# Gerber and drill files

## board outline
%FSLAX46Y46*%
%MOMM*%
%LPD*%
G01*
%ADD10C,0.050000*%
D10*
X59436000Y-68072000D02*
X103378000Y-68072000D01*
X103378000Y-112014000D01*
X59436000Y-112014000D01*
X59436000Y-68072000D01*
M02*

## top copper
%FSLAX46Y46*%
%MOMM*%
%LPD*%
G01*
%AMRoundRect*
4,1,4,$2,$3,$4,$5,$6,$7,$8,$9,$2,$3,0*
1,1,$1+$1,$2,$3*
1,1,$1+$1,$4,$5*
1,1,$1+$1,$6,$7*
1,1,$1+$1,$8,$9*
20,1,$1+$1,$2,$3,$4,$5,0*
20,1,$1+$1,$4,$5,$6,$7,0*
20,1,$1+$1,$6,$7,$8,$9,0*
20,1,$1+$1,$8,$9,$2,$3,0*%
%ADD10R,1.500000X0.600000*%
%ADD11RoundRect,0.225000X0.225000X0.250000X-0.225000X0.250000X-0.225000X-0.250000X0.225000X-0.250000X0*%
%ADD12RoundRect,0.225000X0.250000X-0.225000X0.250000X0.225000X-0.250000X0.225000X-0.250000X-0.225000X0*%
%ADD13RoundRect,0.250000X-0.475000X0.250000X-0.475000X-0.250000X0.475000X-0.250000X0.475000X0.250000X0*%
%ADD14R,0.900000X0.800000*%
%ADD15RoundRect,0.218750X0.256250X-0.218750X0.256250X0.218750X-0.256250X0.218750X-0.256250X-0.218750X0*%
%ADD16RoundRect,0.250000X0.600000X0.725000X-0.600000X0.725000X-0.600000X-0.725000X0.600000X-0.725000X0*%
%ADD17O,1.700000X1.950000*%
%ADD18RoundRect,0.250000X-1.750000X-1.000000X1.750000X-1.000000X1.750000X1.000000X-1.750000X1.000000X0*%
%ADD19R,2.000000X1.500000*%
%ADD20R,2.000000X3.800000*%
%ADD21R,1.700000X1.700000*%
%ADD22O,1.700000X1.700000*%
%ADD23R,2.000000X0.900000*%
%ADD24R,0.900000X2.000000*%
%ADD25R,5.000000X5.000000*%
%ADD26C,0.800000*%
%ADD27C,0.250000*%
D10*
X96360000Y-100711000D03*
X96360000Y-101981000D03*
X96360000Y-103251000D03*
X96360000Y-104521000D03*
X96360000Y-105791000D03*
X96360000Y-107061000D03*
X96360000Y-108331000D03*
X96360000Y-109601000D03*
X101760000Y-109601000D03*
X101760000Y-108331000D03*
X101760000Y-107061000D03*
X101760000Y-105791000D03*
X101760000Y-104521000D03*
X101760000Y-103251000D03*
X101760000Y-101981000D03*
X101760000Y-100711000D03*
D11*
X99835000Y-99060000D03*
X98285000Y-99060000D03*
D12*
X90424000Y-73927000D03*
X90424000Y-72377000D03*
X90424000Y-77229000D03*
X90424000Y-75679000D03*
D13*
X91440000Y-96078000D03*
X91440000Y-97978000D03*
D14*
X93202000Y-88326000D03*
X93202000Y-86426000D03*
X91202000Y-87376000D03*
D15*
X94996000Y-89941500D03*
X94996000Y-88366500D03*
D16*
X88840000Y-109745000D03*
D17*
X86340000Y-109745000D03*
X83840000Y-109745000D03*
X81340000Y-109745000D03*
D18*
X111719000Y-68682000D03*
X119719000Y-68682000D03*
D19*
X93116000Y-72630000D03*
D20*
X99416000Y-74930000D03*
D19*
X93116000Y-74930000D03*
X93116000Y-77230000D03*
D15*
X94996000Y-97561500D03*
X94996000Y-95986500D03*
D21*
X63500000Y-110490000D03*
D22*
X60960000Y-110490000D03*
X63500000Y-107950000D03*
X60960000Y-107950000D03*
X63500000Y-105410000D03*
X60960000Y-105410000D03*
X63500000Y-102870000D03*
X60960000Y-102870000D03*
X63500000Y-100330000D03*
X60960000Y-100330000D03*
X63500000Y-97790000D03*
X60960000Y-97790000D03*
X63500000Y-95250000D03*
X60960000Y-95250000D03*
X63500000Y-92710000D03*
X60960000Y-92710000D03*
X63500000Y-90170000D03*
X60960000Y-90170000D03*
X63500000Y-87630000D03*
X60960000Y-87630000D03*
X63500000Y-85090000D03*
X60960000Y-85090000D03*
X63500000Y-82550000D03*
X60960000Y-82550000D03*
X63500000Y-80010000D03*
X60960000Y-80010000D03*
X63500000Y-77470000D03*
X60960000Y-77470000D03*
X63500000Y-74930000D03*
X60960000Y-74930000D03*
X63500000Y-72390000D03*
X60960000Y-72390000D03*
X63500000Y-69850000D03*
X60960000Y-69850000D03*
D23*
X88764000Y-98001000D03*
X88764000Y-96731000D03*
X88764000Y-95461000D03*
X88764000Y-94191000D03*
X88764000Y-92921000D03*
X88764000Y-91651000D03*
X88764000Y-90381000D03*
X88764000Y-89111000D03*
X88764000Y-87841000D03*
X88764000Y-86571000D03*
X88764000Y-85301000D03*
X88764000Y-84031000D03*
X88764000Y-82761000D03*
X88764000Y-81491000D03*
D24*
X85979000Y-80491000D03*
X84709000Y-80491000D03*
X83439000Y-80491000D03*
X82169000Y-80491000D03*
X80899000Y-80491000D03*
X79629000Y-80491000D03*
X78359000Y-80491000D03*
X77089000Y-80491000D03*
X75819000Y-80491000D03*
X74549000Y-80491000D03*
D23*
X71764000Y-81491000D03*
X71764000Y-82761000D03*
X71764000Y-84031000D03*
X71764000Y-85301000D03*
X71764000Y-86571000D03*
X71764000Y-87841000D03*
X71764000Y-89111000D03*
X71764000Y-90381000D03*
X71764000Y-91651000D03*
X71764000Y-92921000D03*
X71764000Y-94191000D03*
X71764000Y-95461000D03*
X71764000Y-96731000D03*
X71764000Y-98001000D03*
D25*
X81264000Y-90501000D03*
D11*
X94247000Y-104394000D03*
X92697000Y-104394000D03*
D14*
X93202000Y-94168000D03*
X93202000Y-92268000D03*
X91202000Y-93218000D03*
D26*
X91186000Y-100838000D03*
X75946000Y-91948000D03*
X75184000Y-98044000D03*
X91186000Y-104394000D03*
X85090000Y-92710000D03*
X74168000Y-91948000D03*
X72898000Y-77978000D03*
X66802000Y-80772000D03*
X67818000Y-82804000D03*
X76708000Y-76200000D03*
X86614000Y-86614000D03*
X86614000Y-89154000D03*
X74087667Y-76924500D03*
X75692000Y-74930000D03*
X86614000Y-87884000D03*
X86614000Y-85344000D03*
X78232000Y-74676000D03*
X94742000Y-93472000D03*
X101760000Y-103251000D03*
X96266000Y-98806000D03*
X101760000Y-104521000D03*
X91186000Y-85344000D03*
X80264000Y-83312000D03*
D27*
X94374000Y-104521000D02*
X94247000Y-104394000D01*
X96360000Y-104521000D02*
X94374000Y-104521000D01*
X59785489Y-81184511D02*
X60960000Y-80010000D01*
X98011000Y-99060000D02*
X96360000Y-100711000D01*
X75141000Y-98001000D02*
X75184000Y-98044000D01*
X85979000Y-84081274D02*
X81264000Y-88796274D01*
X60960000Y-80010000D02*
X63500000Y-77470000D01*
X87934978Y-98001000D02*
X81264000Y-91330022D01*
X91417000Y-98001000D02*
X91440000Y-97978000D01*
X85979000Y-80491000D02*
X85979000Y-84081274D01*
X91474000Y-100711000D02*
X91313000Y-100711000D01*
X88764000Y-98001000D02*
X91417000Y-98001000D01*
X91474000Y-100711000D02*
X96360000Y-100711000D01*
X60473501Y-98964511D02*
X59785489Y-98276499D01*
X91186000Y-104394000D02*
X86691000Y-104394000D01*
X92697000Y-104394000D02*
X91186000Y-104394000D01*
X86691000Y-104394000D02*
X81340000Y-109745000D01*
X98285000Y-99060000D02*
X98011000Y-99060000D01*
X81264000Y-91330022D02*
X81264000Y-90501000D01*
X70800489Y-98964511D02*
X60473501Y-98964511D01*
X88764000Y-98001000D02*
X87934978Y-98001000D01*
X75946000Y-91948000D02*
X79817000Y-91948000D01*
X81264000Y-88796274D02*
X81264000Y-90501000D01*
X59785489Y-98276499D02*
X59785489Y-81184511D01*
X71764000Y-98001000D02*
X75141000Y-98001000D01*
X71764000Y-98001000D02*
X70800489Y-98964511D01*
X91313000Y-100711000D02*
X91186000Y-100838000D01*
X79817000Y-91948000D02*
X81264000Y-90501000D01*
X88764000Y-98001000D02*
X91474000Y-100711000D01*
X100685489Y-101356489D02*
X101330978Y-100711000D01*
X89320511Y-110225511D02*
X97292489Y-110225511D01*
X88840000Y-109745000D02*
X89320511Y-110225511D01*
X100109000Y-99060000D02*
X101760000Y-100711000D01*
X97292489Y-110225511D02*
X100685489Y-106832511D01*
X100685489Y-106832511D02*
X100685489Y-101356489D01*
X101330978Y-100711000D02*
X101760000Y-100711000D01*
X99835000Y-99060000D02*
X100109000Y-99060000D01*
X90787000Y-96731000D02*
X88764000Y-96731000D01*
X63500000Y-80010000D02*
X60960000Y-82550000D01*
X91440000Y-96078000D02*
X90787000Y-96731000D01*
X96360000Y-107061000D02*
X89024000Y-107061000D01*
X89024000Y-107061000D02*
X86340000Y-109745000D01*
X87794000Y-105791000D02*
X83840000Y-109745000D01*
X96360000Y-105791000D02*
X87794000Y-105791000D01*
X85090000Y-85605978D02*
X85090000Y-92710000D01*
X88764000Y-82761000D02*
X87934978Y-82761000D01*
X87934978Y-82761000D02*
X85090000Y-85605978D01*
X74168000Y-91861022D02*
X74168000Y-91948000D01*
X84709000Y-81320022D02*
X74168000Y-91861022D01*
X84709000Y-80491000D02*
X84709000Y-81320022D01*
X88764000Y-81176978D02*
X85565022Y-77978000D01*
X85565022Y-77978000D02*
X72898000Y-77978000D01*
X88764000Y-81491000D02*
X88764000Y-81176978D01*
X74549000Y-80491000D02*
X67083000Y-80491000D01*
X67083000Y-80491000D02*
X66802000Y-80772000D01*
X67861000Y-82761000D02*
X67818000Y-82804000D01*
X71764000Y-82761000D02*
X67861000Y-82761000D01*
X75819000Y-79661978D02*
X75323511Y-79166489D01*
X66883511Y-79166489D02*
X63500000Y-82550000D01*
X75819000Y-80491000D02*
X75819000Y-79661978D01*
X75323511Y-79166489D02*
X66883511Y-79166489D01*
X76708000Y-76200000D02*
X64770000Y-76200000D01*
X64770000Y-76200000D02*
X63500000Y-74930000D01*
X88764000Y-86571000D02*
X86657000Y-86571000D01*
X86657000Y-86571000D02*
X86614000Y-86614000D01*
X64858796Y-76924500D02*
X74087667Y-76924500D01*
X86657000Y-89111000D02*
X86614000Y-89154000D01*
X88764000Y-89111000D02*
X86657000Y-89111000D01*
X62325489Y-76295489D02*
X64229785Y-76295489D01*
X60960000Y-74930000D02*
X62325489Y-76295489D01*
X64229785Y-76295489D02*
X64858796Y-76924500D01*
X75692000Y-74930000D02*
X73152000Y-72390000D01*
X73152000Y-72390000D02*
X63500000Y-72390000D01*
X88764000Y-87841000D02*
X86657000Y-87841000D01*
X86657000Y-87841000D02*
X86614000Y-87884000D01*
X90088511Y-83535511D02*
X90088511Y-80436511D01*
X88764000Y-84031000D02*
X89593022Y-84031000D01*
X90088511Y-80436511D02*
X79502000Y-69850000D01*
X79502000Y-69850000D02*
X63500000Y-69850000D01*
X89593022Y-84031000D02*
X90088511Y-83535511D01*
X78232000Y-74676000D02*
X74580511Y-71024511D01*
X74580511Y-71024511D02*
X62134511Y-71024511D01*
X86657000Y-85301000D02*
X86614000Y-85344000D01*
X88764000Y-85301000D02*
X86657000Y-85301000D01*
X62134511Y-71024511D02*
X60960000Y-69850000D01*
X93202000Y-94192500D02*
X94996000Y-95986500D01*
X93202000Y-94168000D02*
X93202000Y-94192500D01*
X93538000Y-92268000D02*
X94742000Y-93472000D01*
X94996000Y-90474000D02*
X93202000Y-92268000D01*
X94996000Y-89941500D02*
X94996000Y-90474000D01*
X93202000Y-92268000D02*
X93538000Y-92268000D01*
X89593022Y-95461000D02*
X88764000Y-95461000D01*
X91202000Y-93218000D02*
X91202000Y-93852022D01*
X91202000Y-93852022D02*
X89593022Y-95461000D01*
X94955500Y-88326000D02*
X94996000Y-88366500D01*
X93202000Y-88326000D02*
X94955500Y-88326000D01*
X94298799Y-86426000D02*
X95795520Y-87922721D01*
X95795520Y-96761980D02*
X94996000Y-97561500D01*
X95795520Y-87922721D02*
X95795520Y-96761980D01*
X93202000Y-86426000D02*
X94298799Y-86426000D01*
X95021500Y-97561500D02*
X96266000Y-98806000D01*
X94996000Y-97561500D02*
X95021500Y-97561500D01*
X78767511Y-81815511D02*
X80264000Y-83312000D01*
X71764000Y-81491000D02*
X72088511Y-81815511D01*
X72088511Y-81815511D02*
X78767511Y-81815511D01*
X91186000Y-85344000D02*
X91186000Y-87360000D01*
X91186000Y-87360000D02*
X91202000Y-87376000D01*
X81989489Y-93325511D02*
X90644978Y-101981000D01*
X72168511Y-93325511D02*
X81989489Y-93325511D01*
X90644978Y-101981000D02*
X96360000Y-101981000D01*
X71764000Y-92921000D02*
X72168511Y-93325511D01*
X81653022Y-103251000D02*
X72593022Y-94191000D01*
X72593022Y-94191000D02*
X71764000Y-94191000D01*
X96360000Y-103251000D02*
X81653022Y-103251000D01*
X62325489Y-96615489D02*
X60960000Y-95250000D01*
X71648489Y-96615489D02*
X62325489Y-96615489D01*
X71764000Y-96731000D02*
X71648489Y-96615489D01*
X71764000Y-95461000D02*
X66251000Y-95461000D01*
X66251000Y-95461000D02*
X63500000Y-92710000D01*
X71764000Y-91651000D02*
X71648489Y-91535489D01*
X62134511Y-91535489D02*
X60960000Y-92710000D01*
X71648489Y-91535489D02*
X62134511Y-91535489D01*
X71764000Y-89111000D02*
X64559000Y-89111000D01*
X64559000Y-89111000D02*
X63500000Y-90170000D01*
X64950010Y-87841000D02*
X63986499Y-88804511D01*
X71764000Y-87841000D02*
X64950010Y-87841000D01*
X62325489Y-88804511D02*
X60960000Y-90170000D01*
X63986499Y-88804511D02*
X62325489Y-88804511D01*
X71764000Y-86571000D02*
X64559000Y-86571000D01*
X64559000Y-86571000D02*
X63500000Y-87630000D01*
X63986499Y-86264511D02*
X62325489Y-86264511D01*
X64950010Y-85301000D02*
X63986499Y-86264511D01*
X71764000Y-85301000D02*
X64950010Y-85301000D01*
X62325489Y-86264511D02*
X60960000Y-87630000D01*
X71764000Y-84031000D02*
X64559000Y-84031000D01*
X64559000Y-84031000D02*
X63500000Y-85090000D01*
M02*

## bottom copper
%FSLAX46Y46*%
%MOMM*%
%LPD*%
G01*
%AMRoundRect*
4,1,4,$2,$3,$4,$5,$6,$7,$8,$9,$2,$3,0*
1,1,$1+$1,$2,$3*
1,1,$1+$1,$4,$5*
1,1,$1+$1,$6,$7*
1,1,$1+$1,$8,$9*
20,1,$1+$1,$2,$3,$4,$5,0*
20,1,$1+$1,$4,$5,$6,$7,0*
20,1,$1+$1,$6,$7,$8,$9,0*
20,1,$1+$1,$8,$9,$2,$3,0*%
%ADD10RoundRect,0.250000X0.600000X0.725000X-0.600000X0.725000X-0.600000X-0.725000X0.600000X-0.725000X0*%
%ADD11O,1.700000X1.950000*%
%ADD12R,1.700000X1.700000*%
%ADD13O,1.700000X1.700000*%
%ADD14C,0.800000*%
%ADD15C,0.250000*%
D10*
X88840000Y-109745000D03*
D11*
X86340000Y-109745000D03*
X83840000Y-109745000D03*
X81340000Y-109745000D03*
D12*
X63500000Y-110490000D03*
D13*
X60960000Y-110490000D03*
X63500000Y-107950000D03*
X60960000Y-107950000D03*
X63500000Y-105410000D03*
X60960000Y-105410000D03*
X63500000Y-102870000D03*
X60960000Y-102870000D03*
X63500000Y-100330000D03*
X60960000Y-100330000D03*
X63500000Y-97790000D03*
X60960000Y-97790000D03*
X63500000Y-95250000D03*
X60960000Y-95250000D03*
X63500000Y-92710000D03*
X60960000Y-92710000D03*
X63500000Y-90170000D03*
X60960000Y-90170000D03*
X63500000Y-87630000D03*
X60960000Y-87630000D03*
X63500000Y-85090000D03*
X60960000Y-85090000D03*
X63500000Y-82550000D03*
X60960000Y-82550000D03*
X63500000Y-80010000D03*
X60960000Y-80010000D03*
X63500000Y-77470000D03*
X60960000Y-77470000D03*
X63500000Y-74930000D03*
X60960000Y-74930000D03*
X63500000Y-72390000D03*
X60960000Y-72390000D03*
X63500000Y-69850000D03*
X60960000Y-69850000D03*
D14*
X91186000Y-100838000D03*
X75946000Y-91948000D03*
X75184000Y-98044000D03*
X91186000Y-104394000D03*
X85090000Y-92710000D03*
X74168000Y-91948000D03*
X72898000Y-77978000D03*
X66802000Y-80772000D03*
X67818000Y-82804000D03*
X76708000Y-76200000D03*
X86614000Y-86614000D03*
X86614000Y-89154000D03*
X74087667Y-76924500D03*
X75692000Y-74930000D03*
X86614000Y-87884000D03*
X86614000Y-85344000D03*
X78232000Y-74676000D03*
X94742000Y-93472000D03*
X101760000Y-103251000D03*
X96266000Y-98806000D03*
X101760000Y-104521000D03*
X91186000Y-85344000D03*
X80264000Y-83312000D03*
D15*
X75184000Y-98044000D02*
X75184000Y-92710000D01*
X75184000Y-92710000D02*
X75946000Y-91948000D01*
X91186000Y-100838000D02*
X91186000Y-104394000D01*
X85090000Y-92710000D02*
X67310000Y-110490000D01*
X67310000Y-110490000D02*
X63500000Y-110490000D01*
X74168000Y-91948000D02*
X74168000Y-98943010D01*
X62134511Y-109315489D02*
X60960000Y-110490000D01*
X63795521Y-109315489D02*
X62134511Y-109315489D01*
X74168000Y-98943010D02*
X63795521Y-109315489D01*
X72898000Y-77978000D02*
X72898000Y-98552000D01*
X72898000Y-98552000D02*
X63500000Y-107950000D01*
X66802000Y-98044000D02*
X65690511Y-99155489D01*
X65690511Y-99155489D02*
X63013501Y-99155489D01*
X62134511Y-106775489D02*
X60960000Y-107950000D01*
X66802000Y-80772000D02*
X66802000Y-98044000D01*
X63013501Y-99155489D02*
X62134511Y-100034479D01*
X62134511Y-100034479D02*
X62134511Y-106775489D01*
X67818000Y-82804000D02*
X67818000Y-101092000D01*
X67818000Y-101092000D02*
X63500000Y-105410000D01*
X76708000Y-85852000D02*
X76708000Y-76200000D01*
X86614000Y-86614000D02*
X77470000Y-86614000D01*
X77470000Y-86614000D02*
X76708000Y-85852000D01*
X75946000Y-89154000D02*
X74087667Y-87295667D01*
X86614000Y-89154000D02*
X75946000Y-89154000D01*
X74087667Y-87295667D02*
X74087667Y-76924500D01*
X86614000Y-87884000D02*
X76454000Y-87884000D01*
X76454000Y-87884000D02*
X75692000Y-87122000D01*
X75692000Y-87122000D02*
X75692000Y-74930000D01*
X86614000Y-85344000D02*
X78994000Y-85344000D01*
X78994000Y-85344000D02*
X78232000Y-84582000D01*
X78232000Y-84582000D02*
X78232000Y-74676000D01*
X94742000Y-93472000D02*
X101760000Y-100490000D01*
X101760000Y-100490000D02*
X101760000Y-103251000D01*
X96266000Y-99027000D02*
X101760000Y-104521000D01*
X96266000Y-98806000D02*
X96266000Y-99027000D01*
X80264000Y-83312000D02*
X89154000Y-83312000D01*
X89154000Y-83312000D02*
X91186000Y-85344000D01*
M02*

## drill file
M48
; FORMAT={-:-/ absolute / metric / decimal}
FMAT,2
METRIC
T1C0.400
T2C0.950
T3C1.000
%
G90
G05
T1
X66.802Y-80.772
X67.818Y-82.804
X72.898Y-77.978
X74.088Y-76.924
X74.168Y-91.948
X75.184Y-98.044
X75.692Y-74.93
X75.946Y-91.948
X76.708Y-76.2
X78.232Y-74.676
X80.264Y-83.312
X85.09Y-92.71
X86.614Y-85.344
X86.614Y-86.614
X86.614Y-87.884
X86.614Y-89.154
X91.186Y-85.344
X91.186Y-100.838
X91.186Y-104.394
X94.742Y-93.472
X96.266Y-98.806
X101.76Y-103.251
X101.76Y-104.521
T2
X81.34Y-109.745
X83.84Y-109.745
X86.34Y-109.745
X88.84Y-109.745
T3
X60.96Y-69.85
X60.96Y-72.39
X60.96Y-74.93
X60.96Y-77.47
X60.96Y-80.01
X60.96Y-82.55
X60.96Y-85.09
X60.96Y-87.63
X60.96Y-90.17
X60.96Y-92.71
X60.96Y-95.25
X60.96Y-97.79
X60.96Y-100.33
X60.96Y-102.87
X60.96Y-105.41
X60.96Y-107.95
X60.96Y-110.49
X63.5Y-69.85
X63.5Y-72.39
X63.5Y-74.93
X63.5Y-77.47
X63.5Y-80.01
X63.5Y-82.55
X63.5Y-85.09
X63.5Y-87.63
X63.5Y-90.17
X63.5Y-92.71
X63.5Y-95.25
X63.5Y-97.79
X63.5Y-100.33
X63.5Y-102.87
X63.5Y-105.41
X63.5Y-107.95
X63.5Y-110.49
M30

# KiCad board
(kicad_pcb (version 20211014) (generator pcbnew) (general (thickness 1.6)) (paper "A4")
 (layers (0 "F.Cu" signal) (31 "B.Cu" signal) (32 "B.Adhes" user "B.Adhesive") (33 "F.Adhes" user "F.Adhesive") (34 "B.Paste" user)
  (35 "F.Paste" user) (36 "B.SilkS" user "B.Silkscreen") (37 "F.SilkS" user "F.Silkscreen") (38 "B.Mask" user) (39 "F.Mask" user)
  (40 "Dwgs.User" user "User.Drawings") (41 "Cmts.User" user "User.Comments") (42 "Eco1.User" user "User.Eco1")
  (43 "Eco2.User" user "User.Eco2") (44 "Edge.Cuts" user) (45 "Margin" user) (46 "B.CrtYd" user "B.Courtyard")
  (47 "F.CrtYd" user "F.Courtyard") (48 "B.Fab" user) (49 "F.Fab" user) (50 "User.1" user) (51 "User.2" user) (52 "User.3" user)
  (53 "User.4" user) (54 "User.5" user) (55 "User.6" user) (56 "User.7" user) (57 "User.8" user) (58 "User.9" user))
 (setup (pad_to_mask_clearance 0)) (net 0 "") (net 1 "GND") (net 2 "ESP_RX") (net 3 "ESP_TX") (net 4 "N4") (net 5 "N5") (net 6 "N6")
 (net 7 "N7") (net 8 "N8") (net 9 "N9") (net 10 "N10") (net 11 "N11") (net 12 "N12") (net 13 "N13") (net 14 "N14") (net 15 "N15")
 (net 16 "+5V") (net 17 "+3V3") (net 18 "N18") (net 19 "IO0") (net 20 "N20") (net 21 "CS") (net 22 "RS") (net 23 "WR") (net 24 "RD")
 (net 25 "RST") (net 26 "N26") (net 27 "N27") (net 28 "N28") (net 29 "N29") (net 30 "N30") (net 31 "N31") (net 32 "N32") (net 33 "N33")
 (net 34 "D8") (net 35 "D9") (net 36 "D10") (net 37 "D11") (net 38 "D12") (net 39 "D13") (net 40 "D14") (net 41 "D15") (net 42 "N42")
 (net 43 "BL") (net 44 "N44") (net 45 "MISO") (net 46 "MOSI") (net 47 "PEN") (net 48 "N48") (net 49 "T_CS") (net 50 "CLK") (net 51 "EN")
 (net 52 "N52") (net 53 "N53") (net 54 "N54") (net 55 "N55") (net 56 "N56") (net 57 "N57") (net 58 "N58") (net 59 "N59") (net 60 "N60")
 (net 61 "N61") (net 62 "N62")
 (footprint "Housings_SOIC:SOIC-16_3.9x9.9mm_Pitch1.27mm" (layer "F.Cu") (at 99.06 105.156)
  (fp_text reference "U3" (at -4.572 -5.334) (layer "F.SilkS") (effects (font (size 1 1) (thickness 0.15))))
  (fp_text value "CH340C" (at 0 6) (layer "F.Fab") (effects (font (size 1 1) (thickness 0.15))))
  (pad "1" smd rect locked (at -2.7 -4.445) (size 1.5 0.6) (layers "F.Cu" "F.Paste" "F.Mask") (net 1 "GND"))
  (pad "2" smd rect locked (at -2.7 -3.175) (size 1.5 0.6) (layers "F.Cu" "F.Paste" "F.Mask") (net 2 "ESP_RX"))
  (pad "3" smd rect locked (at -2.7 -1.905) (size 1.5 0.6) (layers "F.Cu" "F.Paste" "F.Mask") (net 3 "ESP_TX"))
  (pad "4" smd rect locked (at -2.7 -0.635) (size 1.5 0.6) (layers "F.Cu" "F.Paste" "F.Mask") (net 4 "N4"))
  (pad "5" smd rect locked (at -2.7 0.635) (size 1.5 0.6) (layers "F.Cu" "F.Paste" "F.Mask") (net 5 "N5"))
  (pad "6" smd rect locked (at -2.7 1.905) (size 1.5 0.6) (layers "F.Cu" "F.Paste" "F.Mask") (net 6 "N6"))
  (pad "7" smd rect locked (at -2.7 3.175) (size 1.5 0.6) (layers "F.Cu" "F.Paste" "F.Mask") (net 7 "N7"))
  (pad "8" smd rect locked (at -2.7 4.445) (size 1.5 0.6) (layers "F.Cu" "F.Paste" "F.Mask") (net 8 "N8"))
  (pad "9" smd rect locked (at 2.7 4.445) (size 1.5 0.6) (layers "F.Cu" "F.Paste" "F.Mask") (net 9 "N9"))
  (pad "10" smd rect locked (at 2.7 3.175) (size 1.5 0.6) (layers "F.Cu" "F.Paste" "F.Mask") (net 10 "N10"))
  (pad "11" smd rect locked (at 2.7 1.905) (size 1.5 0.6) (layers "F.Cu" "F.Paste" "F.Mask") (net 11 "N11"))
  (pad "12" smd rect locked (at 2.7 0.635) (size 1.5 0.6) (layers "F.Cu" "F.Paste" "F.Mask") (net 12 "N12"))
  (pad "13" smd rect locked (at 2.7 -0.635) (size 1.5 0.6) (layers "F.Cu" "F.Paste" "F.Mask") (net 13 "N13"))
  (pad "14" smd rect locked (at 2.7 -1.905) (size 1.5 0.6) (layers "F.Cu" "F.Paste" "F.Mask") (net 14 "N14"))
  (pad "15" smd rect locked (at 2.7 -3.175) (size 1.5 0.6) (layers "F.Cu" "F.Paste" "F.Mask") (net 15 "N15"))
  (pad "16" smd rect locked (at 2.7 -4.445) (size 1.5 0.6) (layers "F.Cu" "F.Paste" "F.Mask") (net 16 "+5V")))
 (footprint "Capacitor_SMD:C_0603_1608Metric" (layer "F.Cu") (at 99.06 99.06 180)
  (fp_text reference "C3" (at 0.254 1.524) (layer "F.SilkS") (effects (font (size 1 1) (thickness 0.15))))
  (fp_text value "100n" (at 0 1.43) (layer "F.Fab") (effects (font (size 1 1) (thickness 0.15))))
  (pad "1" smd roundrect locked (at -0.775 0 180) (size 0.9 0.95) (layers "F.Cu" "F.Paste" "F.Mask") (roundrect_rratio 0.25) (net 16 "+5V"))
  (pad "2" smd roundrect locked (at 0.775 0 180) (size 0.9 0.95) (layers "F.Cu" "F.Paste" "F.Mask") (roundrect_rratio 0.25) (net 1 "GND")))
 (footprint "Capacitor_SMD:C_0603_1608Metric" (layer "F.Cu") (at 90.424 73.152 90)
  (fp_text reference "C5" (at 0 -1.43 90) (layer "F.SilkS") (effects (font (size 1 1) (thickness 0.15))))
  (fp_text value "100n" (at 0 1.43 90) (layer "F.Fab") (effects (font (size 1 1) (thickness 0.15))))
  (pad "1" smd roundrect locked (at -0.775 0 90) (size 0.9 0.95) (layers "F.Cu" "F.Paste" "F.Mask") (roundrect_rratio 0.25) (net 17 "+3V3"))
  (pad "2" smd roundrect locked (at 0.775 0 90) (size 0.9 0.95) (layers "F.Cu" "F.Paste" "F.Mask") (roundrect_rratio 0.25) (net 1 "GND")))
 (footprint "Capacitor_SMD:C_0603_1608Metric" (layer "F.Cu") (at 90.424 76.454 90)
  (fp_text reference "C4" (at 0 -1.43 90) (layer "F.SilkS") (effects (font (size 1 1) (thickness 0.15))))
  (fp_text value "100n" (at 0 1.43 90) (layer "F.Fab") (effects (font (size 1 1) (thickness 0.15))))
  (pad "1" smd roundrect locked (at -0.775 0 90) (size 0.9 0.95) (layers "F.Cu" "F.Paste" "F.Mask") (roundrect_rratio 0.25) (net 16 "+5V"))
  (pad "2" smd roundrect locked (at 0.775 0 90) (size 0.9 0.95) (layers "F.Cu" "F.Paste" "F.Mask") (roundrect_rratio 0.25) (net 1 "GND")))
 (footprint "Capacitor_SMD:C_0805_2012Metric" (layer "F.Cu") (at 91.44 97.028 -90)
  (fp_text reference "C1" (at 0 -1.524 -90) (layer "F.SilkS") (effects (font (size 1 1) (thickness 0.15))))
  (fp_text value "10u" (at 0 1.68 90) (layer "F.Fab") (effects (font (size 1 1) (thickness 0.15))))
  (pad "1" smd roundrect locked (at -0.95 0 270) (size 1 1.45) (layers "F.Cu" "F.Paste" "F.Mask") (roundrect_rratio 0.25) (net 17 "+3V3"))
  (pad "2" smd roundrect locked (at 0.95 0 270) (size 1 1.45) (layers "F.Cu" "F.Paste" "F.Mask") (roundrect_rratio 0.25) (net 1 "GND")))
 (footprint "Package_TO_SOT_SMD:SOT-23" (layer "F.Cu") (at 92.202 87.376 180)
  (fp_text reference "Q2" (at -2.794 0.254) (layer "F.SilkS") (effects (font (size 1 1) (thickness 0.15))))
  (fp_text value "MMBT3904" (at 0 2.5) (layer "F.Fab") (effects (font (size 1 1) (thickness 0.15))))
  (pad "1" smd rect locked (at -1 -0.95 180) (size 0.9 0.8) (layers "F.Cu" "F.Paste" "F.Mask") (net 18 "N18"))
  (pad "2" smd rect locked (at -1 0.95 180) (size 0.9 0.8) (layers "F.Cu" "F.Paste" "F.Mask") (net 13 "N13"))
  (pad "3" smd rect locked (at 1 0 180) (size 0.9 0.8) (layers "F.Cu" "F.Paste" "F.Mask") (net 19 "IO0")))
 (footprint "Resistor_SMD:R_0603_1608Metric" (layer "F.Cu") (at 94.996 89.154 90)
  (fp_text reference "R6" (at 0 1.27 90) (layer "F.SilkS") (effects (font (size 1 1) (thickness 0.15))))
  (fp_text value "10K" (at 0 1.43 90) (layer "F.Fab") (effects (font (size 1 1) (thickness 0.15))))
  (pad "1" smd roundrect locked (at -0.7875 0 90) (size 0.875 0.95) (layers "F.Cu" "F.Paste" "F.Mask") (roundrect_rratio 0.25)
   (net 14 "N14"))
  (pad "2" smd roundrect locked (at 0.7875 0 90) (size 0.875 0.95) (layers "F.Cu" "F.Paste" "F.Mask") (roundrect_rratio 0.25) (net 18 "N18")))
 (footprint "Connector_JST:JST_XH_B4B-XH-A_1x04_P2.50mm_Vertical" (layer "F.Cu") (at 88.84 109.745 180)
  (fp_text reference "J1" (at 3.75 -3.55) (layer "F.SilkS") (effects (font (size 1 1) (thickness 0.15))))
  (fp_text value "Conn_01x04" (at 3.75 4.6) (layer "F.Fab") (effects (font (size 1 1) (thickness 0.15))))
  (pad "1" thru_hole roundrect (at 0 0 180) (size 1.7 1.95) (drill 0.95) (layers *.Cu *.Mask) (roundrect_rratio 0.147059) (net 16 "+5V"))
  (pad "2" thru_hole oval (at 2.5 0 180) (size 1.7 1.95) (drill 0.95) (layers *.Cu *.Mask) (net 6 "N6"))
  (pad "3" thru_hole oval (at 5 0 180) (size 1.7 1.95) (drill 0.95) (layers *.Cu *.Mask) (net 5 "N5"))
  (pad "4" thru_hole oval (at 7.5 0 180) (size 1.7 1.95) (drill 0.95) (layers *.Cu *.Mask) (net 1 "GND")))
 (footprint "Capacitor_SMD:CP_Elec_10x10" (layer "F.Cu") (at 115.719 68.682)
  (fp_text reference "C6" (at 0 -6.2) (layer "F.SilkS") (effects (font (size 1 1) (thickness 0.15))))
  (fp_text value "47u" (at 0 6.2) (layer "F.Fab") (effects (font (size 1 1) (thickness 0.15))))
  (pad "1" smd roundrect locked (at -4 0) (size 4 2.5) (layers "F.Cu" "F.Paste" "F.Mask") (roundrect_rratio 0.1) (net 16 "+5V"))
  (pad "2" smd roundrect locked (at 4 0) (size 4 2.5) (layers "F.Cu" "F.Paste" "F.Mask") (roundrect_rratio 0.1) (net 1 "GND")))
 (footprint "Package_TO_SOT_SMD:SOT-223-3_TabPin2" (layer "F.Cu") (at 96.266 74.93)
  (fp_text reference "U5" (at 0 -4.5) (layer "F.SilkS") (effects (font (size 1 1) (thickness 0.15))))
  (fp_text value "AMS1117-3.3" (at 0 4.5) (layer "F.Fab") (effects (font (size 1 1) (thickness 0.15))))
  (pad "1" smd rect locked (at -3.15 -2.3) (size 2 1.5) (layers "F.Cu" "F.Paste" "F.Mask") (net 1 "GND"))
  (pad "2" smd rect locked (at 3.15 0) (size 2 3.8) (layers "F.Cu" "F.Paste" "F.Mask") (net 17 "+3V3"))
  (pad "2" smd rect locked (at -3.15 0) (size 2 1.5) (layers "F.Cu" "F.Paste" "F.Mask") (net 17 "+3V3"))
  (pad "3" smd rect locked (at -3.15 2.3) (size 2 1.5) (layers "F.Cu" "F.Paste" "F.Mask") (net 16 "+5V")))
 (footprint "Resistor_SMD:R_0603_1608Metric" (layer "F.Cu") (at 94.996 96.774 90)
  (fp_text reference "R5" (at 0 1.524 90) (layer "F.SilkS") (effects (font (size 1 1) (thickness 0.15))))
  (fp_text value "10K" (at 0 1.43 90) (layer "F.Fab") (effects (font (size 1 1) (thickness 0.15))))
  (pad "1" smd roundrect locked (at -0.7875 0 90) (size 0.875 0.95) (layers "F.Cu" "F.Paste" "F.Mask") (roundrect_rratio 0.25)
   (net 13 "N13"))
  (pad "2" smd roundrect locked (at 0.7875 0 90) (size 0.875 0.95) (layers "F.Cu" "F.Paste" "F.Mask") (roundrect_rratio 0.25) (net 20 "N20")))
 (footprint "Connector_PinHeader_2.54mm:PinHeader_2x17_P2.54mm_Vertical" (layer "F.Cu") (at 63.5 110.49 180)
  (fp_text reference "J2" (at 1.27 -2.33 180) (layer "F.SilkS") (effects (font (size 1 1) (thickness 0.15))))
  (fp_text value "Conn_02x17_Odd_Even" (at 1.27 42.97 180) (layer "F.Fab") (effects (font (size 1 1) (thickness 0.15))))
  (pad "1" thru_hole rect locked (at 0 0 180) (size 1.7 1.7) (drill 1) (layers *.Cu *.Mask) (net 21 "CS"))
  (pad "2" thru_hole oval locked (at 2.54 0 180) (size 1.7 1.7) (drill 1) (layers *.Cu *.Mask) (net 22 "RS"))
  (pad "3" thru_hole oval locked (at 0 2.54 180) (size 1.7 1.7) (drill 1) (layers *.Cu *.Mask) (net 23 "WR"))
  (pad "4" thru_hole oval locked (at 2.54 2.54 180) (size 1.7 1.7) (drill 1) (layers *.Cu *.Mask) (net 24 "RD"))
  (pad "5" thru_hole oval locked (at 0 5.08 180) (size 1.7 1.7) (drill 1) (layers *.Cu *.Mask) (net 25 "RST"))
  (pad "6" thru_hole oval locked (at 2.54 5.08 180) (size 1.7 1.7) (drill 1) (layers *.Cu *.Mask) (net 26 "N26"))
  (pad "7" thru_hole oval locked (at 0 7.62 180) (size 1.7 1.7) (drill 1) (layers *.Cu *.Mask) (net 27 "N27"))
  (pad "8" thru_hole oval locked (at 2.54 7.62 180) (size 1.7 1.7) (drill 1) (layers *.Cu *.Mask) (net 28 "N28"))
  (pad "9" thru_hole oval locked (at 0 10.16 180) (size 1.7 1.7) (drill 1) (layers *.Cu *.Mask) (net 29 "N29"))
  (pad "10" thru_hole oval locked (at 2.54 10.16 180) (size 1.7 1.7) (drill 1) (layers *.Cu *.Mask) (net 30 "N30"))
  (pad "11" thru_hole oval locked (at 0 12.7 180) (size 1.7 1.7) (drill 1) (layers *.Cu *.Mask) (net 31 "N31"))
  (pad "12" thru_hole oval locked (at 2.54 12.7 180) (size 1.7 1.7) (drill 1) (layers *.Cu *.Mask) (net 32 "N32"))
  (pad "13" thru_hole oval locked (at 0 15.24 180) (size 1.7 1.7) (drill 1) (layers *.Cu *.Mask) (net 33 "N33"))
  (pad "14" thru_hole oval locked (at 2.54 15.24 180) (size 1.7 1.7) (drill 1) (layers *.Cu *.Mask) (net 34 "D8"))
  (pad "15" thru_hole oval locked (at 0 17.78 180) (size 1.7 1.7) (drill 1) (layers *.Cu *.Mask) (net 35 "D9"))
  (pad "16" thru_hole oval locked (at 2.54 17.78 180) (size 1.7 1.7) (drill 1) (layers *.Cu *.Mask) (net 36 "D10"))
  (pad "17" thru_hole oval locked (at 0 20.32 180) (size 1.7 1.7) (drill 1) (layers *.Cu *.Mask) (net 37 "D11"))
  (pad "18" thru_hole oval locked (at 2.54 20.32 180) (size 1.7 1.7) (drill 1) (layers *.Cu *.Mask) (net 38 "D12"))
  (pad "19" thru_hole oval locked (at 0 22.86 180) (size 1.7 1.7) (drill 1) (layers *.Cu *.Mask) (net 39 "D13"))
  (pad "20" thru_hole oval locked (at 2.54 22.86 180) (size 1.7 1.7) (drill 1) (layers *.Cu *.Mask) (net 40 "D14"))
  (pad "21" thru_hole oval locked (at 0 25.4 180) (size 1.7 1.7) (drill 1) (layers *.Cu *.Mask) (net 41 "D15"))
  (pad "22" thru_hole oval locked (at 2.54 25.4 180) (size 1.7 1.7) (drill 1) (layers *.Cu *.Mask) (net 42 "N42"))
  (pad "23" thru_hole oval locked (at 0 27.94 180) (size 1.7 1.7) (drill 1) (layers *.Cu *.Mask) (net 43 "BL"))
  (pad "24" thru_hole oval locked (at 2.54 27.94 180) (size 1.7 1.7) (drill 1) (layers *.Cu *.Mask) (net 17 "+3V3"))
  (pad "25" thru_hole oval locked (at 0 30.48 180) (size 1.7 1.7) (drill 1) (layers *.Cu *.Mask) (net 17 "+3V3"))
  (pad "26" thru_hole oval locked (at 2.54 30.48 180) (size 1.7 1.7) (drill 1) (layers *.Cu *.Mask) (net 1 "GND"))
  (pad "27" thru_hole oval locked (at 0 33.02 180) (size 1.7 1.7) (drill 1) (layers *.Cu *.Mask) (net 1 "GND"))
  (pad "28" thru_hole oval locked (at 2.54 33.02 180) (size 1.7 1.7) (drill 1) (layers *.Cu *.Mask) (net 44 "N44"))
  (pad "29" thru_hole oval locked (at 0 35.56 180) (size 1.7 1.7) (drill 1) (layers *.Cu *.Mask) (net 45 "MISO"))
  (pad "30" thru_hole oval locked (at 2.54 35.56 180) (size 1.7 1.7) (drill 1) (layers *.Cu *.Mask) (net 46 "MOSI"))
  (pad "31" thru_hole oval locked (at 0 38.1 180) (size 1.7 1.7) (drill 1) (layers *.Cu *.Mask) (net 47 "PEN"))
  (pad "32" thru_hole oval locked (at 2.54 38.1 180) (size 1.7 1.7) (drill 1) (layers *.Cu *.Mask) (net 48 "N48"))
  (pad "33" thru_hole oval locked (at 0 40.64 180) (size 1.7 1.7) (drill 1) (layers *.Cu *.Mask) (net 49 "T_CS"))
  (pad "34" thru_hole oval locked (at 2.54 40.64 180) (size 1.7 1.7) (drill 1) (layers *.Cu *.Mask) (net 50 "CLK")))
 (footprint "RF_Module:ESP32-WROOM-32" (layer "F.Cu") (at 80.264 89.746 180)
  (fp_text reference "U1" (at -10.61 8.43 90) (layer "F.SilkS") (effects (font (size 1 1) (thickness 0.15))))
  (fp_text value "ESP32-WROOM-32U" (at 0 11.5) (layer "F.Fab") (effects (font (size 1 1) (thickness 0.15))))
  (pad "1" smd rect locked (at -8.5 -8.255 180) (size 2 0.9) (layers "F.Cu" "F.Paste" "F.Mask") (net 1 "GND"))
  (pad "2" smd rect locked (at -8.5 -6.985 180) (size 2 0.9) (layers "F.Cu" "F.Paste" "F.Mask") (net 17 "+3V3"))
  (pad "3" smd rect locked (at -8.5 -5.715 180) (size 2 0.9) (layers "F.Cu" "F.Paste" "F.Mask") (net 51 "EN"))
  (pad "4" smd rect locked (at -8.5 -4.445 180) (size 2 0.9) (layers "F.Cu" "F.Paste" "F.Mask") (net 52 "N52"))
  (pad "5" smd rect locked (at -8.5 -3.175 180) (size 2 0.9) (layers "F.Cu" "F.Paste" "F.Mask") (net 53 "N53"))
  (pad "6" smd rect locked (at -8.5 -1.905 180) (size 2 0.9) (layers "F.Cu" "F.Paste" "F.Mask") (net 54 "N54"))
  (pad "7" smd rect locked (at -8.5 -0.635 180) (size 2 0.9) (layers "F.Cu" "F.Paste" "F.Mask") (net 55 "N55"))
  (pad "8" smd rect locked (at -8.5 0.635 180) (size 2 0.9) (layers "F.Cu" "F.Paste" "F.Mask") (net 46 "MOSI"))
  (pad "9" smd rect locked (at -8.5 1.905 180) (size 2 0.9) (layers "F.Cu" "F.Paste" "F.Mask") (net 47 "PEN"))
  (pad "10" smd rect locked (at -8.5 3.175 180) (size 2 0.9) (layers "F.Cu" "F.Paste" "F.Mask") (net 45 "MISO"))
  (pad "11" smd rect locked (at -8.5 4.445 180) (size 2 0.9) (layers "F.Cu" "F.Paste" "F.Mask") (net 50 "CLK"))
  (pad "12" smd rect locked (at -8.5 5.715 180) (size 2 0.9) (layers "F.Cu" "F.Paste" "F.Mask") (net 49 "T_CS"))
  (pad "13" smd rect locked (at -8.5 6.985 180) (size 2 0.9) (layers "F.Cu" "F.Paste" "F.Mask") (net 21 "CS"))
  (pad "14" smd rect locked (at -8.5 8.255 180) (size 2 0.9) (layers "F.Cu" "F.Paste" "F.Mask") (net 23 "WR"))
  (pad "15" smd rect locked (at -5.715 9.255 270) (size 2 0.9) (layers "F.Cu" "F.Paste" "F.Mask") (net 1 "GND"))
  (pad "16" smd rect locked (at -4.445 9.255 270) (size 2 0.9) (layers "F.Cu" "F.Paste" "F.Mask") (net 22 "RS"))
  (pad "17" smd rect locked (at -3.175 9.255 270) (size 2 0.9) (layers "F.Cu" "F.Paste" "F.Mask") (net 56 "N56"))
  (pad "18" smd rect locked (at -1.905 9.255 270) (size 2 0.9) (layers "F.Cu" "F.Paste" "F.Mask") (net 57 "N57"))
  (pad "19" smd rect locked (at -0.635 9.255 270) (size 2 0.9) (layers "F.Cu" "F.Paste" "F.Mask") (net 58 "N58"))
  (pad "20" smd rect locked (at 0.635 9.255 270) (size 2 0.9) (layers "F.Cu" "F.Paste" "F.Mask") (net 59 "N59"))
  (pad "21" smd rect locked (at 1.905 9.255 270) (size 2 0.9) (layers "F.Cu" "F.Paste" "F.Mask") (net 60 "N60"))
  (pad "22" smd rect locked (at 3.175 9.255 270) (size 2 0.9) (layers "F.Cu" "F.Paste" "F.Mask") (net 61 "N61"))
  (pad "23" smd rect locked (at 4.445 9.255 270) (size 2 0.9) (layers "F.Cu" "F.Paste" "F.Mask") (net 43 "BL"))
  (pad "24" smd rect locked (at 5.715 9.255 270) (size 2 0.9) (layers "F.Cu" "F.Paste" "F.Mask") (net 24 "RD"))
  (pad "25" smd rect locked (at 8.5 8.255 180) (size 2 0.9) (layers "F.Cu" "F.Paste" "F.Mask") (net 19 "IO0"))
  (pad "26" smd rect locked (at 8.5 6.985 180) (size 2 0.9) (layers "F.Cu" "F.Paste" "F.Mask") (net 25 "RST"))
  (pad "27" smd rect locked (at 8.5 5.715 180) (size 2 0.9) (layers "F.Cu" "F.Paste" "F.Mask") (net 41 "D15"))
  (pad "28" smd rect locked (at 8.5 4.445 180) (size 2 0.9) (layers "F.Cu" "F.Paste" "F.Mask") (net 40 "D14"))
  (pad "29" smd rect locked (at 8.5 3.175 180) (size 2 0.9) (layers "F.Cu" "F.Paste" "F.Mask") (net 39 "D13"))
  (pad "30" smd rect locked (at 8.5 1.905 180) (size 2 0.9) (layers "F.Cu" "F.Paste" "F.Mask") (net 38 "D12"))
  (pad "31" smd rect locked (at 8.5 0.635 180) (size 2 0.9) (layers "F.Cu" "F.Paste" "F.Mask") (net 37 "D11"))
  (pad "32" smd rect locked (at 8.5 -0.635 180) (size 2 0.9) (layers "F.Cu" "F.Paste" "F.Mask") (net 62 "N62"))
  (pad "33" smd rect locked (at 8.5 -1.905 180) (size 2 0.9) (layers "F.Cu" "F.Paste" "F.Mask") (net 36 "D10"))
  (pad "34" smd rect locked (at 8.5 -3.175 180) (size 2 0.9) (layers "F.Cu" "F.Paste" "F.Mask") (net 2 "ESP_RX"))
  (pad "35" smd rect locked (at 8.5 -4.445 180) (size 2 0.9) (layers "F.Cu" "F.Paste" "F.Mask") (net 3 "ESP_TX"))
  (pad "36" smd rect locked (at 8.5 -5.715 180) (size 2 0.9) (layers "F.Cu" "F.Paste" "F.Mask") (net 35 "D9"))
  (pad "37" smd rect locked (at 8.5 -6.985 180) (size 2 0.9) (layers "F.Cu" "F.Paste" "F.Mask") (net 34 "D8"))
  (pad "38" smd rect locked (at 8.5 -8.255 180) (size 2 0.9) (layers "F.Cu" "F.Paste" "F.Mask") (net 1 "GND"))
  (pad "39" smd rect locked (at -1 -0.755 180) (size 5 5) (layers "F.Cu" "F.Paste" "F.Mask") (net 1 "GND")))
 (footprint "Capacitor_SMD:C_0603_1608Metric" (layer "F.Cu") (at 93.472 104.394 180)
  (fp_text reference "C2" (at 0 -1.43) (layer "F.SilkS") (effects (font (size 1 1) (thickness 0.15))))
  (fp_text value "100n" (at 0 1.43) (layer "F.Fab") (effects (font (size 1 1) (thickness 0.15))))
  (pad "1" smd roundrect locked (at -0.775 0 180) (size 0.9 0.95) (layers "F.Cu" "F.Paste" "F.Mask") (roundrect_rratio 0.25) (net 4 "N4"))
  (pad "2" smd roundrect locked (at 0.775 0 180) (size 0.9 0.95) (layers "F.Cu" "F.Paste" "F.Mask") (roundrect_rratio 0.25) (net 1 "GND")))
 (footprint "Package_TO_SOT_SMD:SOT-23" (layer "F.Cu") (at 92.202 93.218 180)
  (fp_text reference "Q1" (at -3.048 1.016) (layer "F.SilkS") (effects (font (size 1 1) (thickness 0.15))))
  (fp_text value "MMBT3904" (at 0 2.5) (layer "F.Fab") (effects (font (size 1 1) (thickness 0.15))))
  (pad "1" smd rect locked (at -1 -0.95 180) (size 0.9 0.8) (layers "F.Cu" "F.Paste" "F.Mask") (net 20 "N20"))
  (pad "2" smd rect locked (at -1 0.95 180) (size 0.9 0.8) (layers "F.Cu" "F.Paste" "F.Mask") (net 14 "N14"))
  (pad "3" smd rect locked (at 1 0 180) (size 0.9 0.8) (layers "F.Cu" "F.Paste" "F.Mask") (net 51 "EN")))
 (gr_rect (start 59.436 112.014) (end 103.378 68.072) (layer "Edge.Cuts") (width 0.05) (fill none))
 (segment (start 94.374 104.521) (end 94.247 104.394) (width 0.25) (layer "F.Cu") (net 4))
 (segment (start 96.36 104.521) (end 94.374 104.521) (width 0.25) (layer "F.Cu") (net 4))
 (segment (start 59.785489 81.184511) (end 60.96 80.01) (width 0.25) (layer "F.Cu") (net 1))
 (segment (start 98.011 99.06) (end 96.36 100.711) (width 0.25) (layer "F.Cu") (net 1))
 (segment (start 75.141 98.001) (end 75.184 98.044) (width 0.25) (layer "F.Cu") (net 1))
 (segment (start 85.979 84.081274) (end 81.264 88.796274) (width 0.25) (layer "F.Cu") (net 1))
 (segment (start 60.96 80.01) (end 63.5 77.47) (width 0.25) (layer "F.Cu") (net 1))
 (segment (start 87.934978 98.001) (end 81.264 91.330022) (width 0.25) (layer "F.Cu") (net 1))
 (segment (start 91.417 98.001) (end 91.44 97.978) (width 0.25) (layer "F.Cu") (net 1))
 (segment (start 85.979 80.491) (end 85.979 84.081274) (width 0.25) (layer "F.Cu") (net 1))
 (segment (start 91.474 100.711) (end 91.313 100.711) (width 0.25) (layer "F.Cu") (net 1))
 (segment (start 88.764 98.001) (end 91.417 98.001) (width 0.25) (layer "F.Cu") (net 1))
 (segment (start 91.474 100.711) (end 96.36 100.711) (width 0.25) (layer "F.Cu") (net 1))
 (segment (start 60.473501 98.964511) (end 59.785489 98.276499) (width 0.25) (layer "F.Cu") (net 1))
 (segment (start 91.186 104.394) (end 86.691 104.394) (width 0.25) (layer "F.Cu") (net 1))
 (segment (start 92.697 104.394) (end 91.186 104.394) (width 0.25) (layer "F.Cu") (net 1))
 (segment (start 86.691 104.394) (end 81.34 109.745) (width 0.25) (layer "F.Cu") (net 1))
 (segment (start 98.285 99.06) (end 98.011 99.06) (width 0.25) (layer "F.Cu") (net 1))
 (segment (start 81.264 91.330022) (end 81.264 90.501) (width 0.25) (layer "F.Cu") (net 1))
 (segment (start 70.800489 98.964511) (end 60.473501 98.964511) (width 0.25) (layer "F.Cu") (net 1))
 (segment (start 88.764 98.001) (end 87.934978 98.001) (width 0.25) (layer "F.Cu") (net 1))
 (segment (start 75.946 91.948) (end 79.817 91.948) (width 0.25) (layer "F.Cu") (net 1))
 (segment (start 81.264 88.796274) (end 81.264 90.501) (width 0.25) (layer "F.Cu") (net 1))
 (segment (start 59.785489 98.276499) (end 59.785489 81.184511) (width 0.25) (layer "F.Cu") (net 1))
 (segment (start 71.764 98.001) (end 75.141 98.001) (width 0.25) (layer "F.Cu") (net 1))
 (segment (start 71.764 98.001) (end 70.800489 98.964511) (width 0.25) (layer "F.Cu") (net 1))
 (segment (start 91.313 100.711) (end 91.186 100.838) (width 0.25) (layer "F.Cu") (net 1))
 (segment (start 79.817 91.948) (end 81.264 90.501) (width 0.25) (layer "F.Cu") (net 1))
 (segment (start 88.764 98.001) (end 91.474 100.711) (width 0.25) (layer "F.Cu") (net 1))
 (via (at 91.186 100.838) (size 0.8) (drill 0.4) (layers "F.Cu" "B.Cu") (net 1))
 (via (at 75.946 91.948) (size 0.8) (drill 0.4) (layers "F.Cu" "B.Cu") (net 1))
 (via (at 75.184 98.044) (size 0.8) (drill 0.4) (layers "F.Cu" "B.Cu") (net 1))
 (via (at 91.186 104.394) (size 0.8) (drill 0.4) (layers "F.Cu" "B.Cu") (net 1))
 (segment (start 75.184 98.044) (end 75.184 92.71) (width 0.25) (layer "B.Cu") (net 1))
 (segment (start 75.184 92.71) (end 75.946 91.948) (width 0.25) (layer "B.Cu") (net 1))
 (segment (start 91.186 100.838) (end 91.186 104.394) (width 0.25) (layer "B.Cu") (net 1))
 (segment (start 100.685489 101.356489) (end 101.330978 100.711) (width 0.25) (layer "F.Cu") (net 16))
 (segment (start 89.320511 110.225511) (end 97.292489 110.225511) (width 0.25) (layer "F.Cu") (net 16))
 (segment (start 88.84 109.745) (end 89.320511 110.225511) (width 0.25) (layer "F.Cu") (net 16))
 (segment (start 100.109 99.06) (end 101.76 100.711) (width 0.25) (layer "F.Cu") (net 16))
 (segment (start 97.292489 110.225511) (end 100.685489 106.832511) (width 0.25) (layer "F.Cu") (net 16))
 (segment (start 100.685489 106.832511) (end 100.685489 101.356489) (width 0.25) (layer "F.Cu") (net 16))
 (segment (start 101.330978 100.711) (end 101.76 100.711) (width 0.25) (layer "F.Cu") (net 16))
 (segment (start 99.835 99.06) (end 100.109 99.06) (width 0.25) (layer "F.Cu") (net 16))
 (segment (start 90.787 96.731) (end 88.764 96.731) (width 0.25) (layer "F.Cu") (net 17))
 (segment (start 63.5 80.01) (end 60.96 82.55) (width 0.25) (layer "F.Cu") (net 17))
 (segment (start 91.44 96.078) (end 90.787 96.731) (width 0.25) (layer "F.Cu") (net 17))
 (segment (start 96.36 107.061) (end 89.024 107.061) (width 0.25) (layer "F.Cu") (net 6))
 (segment (start 89.024 107.061) (end 86.34 109.745) (width 0.25) (layer "F.Cu") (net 6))
 (segment (start 87.794 105.791) (end 83.84 109.745) (width 0.25) (layer "F.Cu") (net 5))
 (segment (start 96.36 105.791) (end 87.794 105.791) (width 0.25) (layer "F.Cu") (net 5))
 (segment (start 85.09 85.605978) (end 85.09 92.71) (width 0.25) (layer "F.Cu") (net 21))
 (segment (start 88.764 82.761) (end 87.934978 82.761) (width 0.25) (layer "F.Cu") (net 21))
 (segment (start 87.934978 82.761) (end 85.09 85.605978) (width 0.25) (layer "F.Cu") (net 21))
 (via (at 85.09 92.71) (size 0.8) (drill 0.4) (layers "F.Cu" "B.Cu") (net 21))
 (segment (start 85.09 92.71) (end 67.31 110.49) (width 0.25) (layer "B.Cu") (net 21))
 (segment (start 67.31 110.49) (end 63.5 110.49) (width 0.25) (layer "B.Cu") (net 21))
 (segment (start 74.168 91.861022) (end 74.168 91.948) (width 0.25) (layer "F.Cu") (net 22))
 (segment (start 84.709 81.320022) (end 74.168 91.861022) (width 0.25) (layer "F.Cu") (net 22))
 (segment (start 84.709 80.491) (end 84.709 81.320022) (width 0.25) (layer "F.Cu") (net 22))
 (via (at 74.168 91.948) (size 0.8) (drill 0.4) (layers "F.Cu" "B.Cu") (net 22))
 (segment (start 74.168 91.948) (end 74.168 98.94301) (width 0.25) (layer "B.Cu") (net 22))
 (segment (start 62.134511 109.315489) (end 60.96 110.49) (width 0.25) (layer "B.Cu") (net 22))
 (segment (start 63.795521 109.315489) (end 62.134511 109.315489) (width 0.25) (layer "B.Cu") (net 22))
 (segment (start 74.168 98.94301) (end 63.795521 109.315489) (width 0.25) (layer "B.Cu") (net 22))
 (segment (start 88.764 81.176978) (end 85.565022 77.978) (width 0.25) (layer "F.Cu") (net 23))
 (segment (start 85.565022 77.978) (end 72.898 77.978) (width 0.25) (layer "F.Cu") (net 23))
 (segment (start 88.764 81.491) (end 88.764 81.176978) (width 0.25) (layer "F.Cu") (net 23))
 (via (at 72.898 77.978) (size 0.8) (drill 0.4) (layers "F.Cu" "B.Cu") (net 23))
 (segment (start 72.898 77.978) (end 72.898 98.552) (width 0.25) (layer "B.Cu") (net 23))
 (segment (start 72.898 98.552) (end 63.5 107.95) (width 0.25) (layer "B.Cu") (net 23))
 (segment (start 74.549 80.491) (end 67.083 80.491) (width 0.25) (layer "F.Cu") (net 24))
 (segment (start 67.083 80.491) (end 66.802 80.772) (width 0.25) (layer "F.Cu") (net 24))
 (via (at 66.802 80.772) (size 0.8) (drill 0.4) (layers "F.Cu" "B.Cu") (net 24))
 (segment (start 66.802 98.044) (end 65.690511 99.155489) (width 0.25) (layer "B.Cu") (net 24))
 (segment (start 65.690511 99.155489) (end 63.013501 99.155489) (width 0.25) (layer "B.Cu") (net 24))
 (segment (start 62.134511 106.775489) (end 60.96 107.95) (width 0.25) (layer "B.Cu") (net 24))
 (segment (start 66.802 80.772) (end 66.802 98.044) (width 0.25) (layer "B.Cu") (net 24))
 (segment (start 63.013501 99.155489) (end 62.134511 100.034479) (width 0.25) (layer "B.Cu") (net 24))
 (segment (start 62.134511 100.034479) (end 62.134511 106.775489) (width 0.25) (layer "B.Cu") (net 24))
 (segment (start 67.861 82.761) (end 67.818 82.804) (width 0.25) (layer "F.Cu") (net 25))
 (segment (start 71.764 82.761) (end 67.861 82.761) (width 0.25) (layer "F.Cu") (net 25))
 (via (at 67.818 82.804) (size 0.8) (drill 0.4) (layers "F.Cu" "B.Cu") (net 25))
 (segment (start 67.818 82.804) (end 67.818 101.092) (width 0.25) (layer "B.Cu") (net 25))
 (segment (start 67.818 101.092) (end 63.5 105.41) (width 0.25) (layer "B.Cu") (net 25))
 (segment (start 75.819 79.661978) (end 75.323511 79.166489) (width 0.25) (layer "F.Cu") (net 43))
 (segment (start 66.883511 79.166489) (end 63.5 82.55) (width 0.25) (layer "F.Cu") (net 43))
 (segment (start 75.819 80.491) (end 75.819 79.661978) (width 0.25) (layer "F.Cu") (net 43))
 (segment (start 75.323511 79.166489) (end 66.883511 79.166489) (width 0.25) (layer "F.Cu") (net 43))
 (segment (start 76.708 76.2) (end 64.77 76.2) (width 0.25) (layer "F.Cu") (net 45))
 (segment (start 64.77 76.2) (end 63.5 74.93) (width 0.25) (layer "F.Cu") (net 45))
 (segment (start 88.764 86.571) (end 86.657 86.571) (width 0.25) (layer "F.Cu") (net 45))
 (segment (start 86.657 86.571) (end 86.614 86.614) (width 0.25) (layer "F.Cu") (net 45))
 (via (at 76.708 76.2) (size 0.8) (drill 0.4) (layers "F.Cu" "B.Cu") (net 45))
 (via (at 86.614 86.614) (size 0.8) (drill 0.4) (layers "F.Cu" "B.Cu") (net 45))
 (segment (start 76.708 85.852) (end 76.708 76.2) (width 0.25) (layer "B.Cu") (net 45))
 (segment (start 86.614 86.614) (end 77.47 86.614) (width 0.25) (layer "B.Cu") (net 45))
 (segment (start 77.47 86.614) (end 76.708 85.852) (width 0.25) (layer "B.Cu") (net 45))
 (segment (start 64.858796 76.9245) (end 74.087667 76.9245) (width 0.25) (layer "F.Cu") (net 46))
 (segment (start 86.657 89.111) (end 86.614 89.154) (width 0.25) (layer "F.Cu") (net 46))
 (segment (start 88.764 89.111) (end 86.657 89.111) (width 0.25) (layer "F.Cu") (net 46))
 (segment (start 62.325489 76.295489) (end 64.229785 76.295489) (width 0.25) (layer "F.Cu") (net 46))
 (segment (start 60.96 74.93) (end 62.325489 76.295489) (width 0.25) (layer "F.Cu") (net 46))
 (segment (start 64.229785 76.295489) (end 64.858796 76.9245) (width 0.25) (layer "F.Cu") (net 46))
 (via (at 86.614 89.154) (size 0.8) (drill 0.4) (layers "F.Cu" "B.Cu") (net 46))
 (via (at 74.087667 76.9245) (size 0.8) (drill 0.4) (layers "F.Cu" "B.Cu") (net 46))
 (segment (start 75.946 89.154) (end 74.087667 87.295667) (width 0.25) (layer "B.Cu") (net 46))
 (segment (start 86.614 89.154) (end 75.946 89.154) (width 0.25) (layer "B.Cu") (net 46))
 (segment (start 74.087667 87.295667) (end 74.087667 76.9245) (width 0.25) (layer "B.Cu") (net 46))
 (segment (start 75.692 74.93) (end 73.152 72.39) (width 0.25) (layer "F.Cu") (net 47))
 (segment (start 73.152 72.39) (end 63.5 72.39) (width 0.25) (layer "F.Cu") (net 47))
 (segment (start 88.764 87.841) (end 86.657 87.841) (width 0.25) (layer "F.Cu") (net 47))
 (segment (start 86.657 87.841) (end 86.614 87.884) (width 0.25) (layer "F.Cu") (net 47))
 (via (at 75.692 74.93) (size 0.8) (drill 0.4) (layers "F.Cu" "B.Cu") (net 47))
 (via (at 86.614 87.884) (size 0.8) (drill 0.4) (layers "F.Cu" "B.Cu") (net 47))
 (segment (start 86.614 87.884) (end 76.454 87.884) (width 0.25) (layer "B.Cu") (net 47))
 (segment (start 76.454 87.884) (end 75.692 87.122) (width 0.25) (layer "B.Cu") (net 47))
 (segment (start 75.692 87.122) (end 75.692 74.93) (width 0.25) (layer "B.Cu") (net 47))
 (segment (start 90.088511 83.535511) (end 90.088511 80.436511) (width 0.25) (layer "F.Cu") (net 49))
 (segment (start 88.764 84.031) (end 89.593022 84.031) (width 0.25) (layer "F.Cu") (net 49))
 (segment (start 90.088511 80.436511) (end 79.502 69.85) (width 0.25) (layer "F.Cu") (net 49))
 (segment (start 79.502 69.85) (end 63.5 69.85) (width 0.25) (layer "F.Cu") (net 49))
 (segment (start 89.593022 84.031) (end 90.088511 83.535511) (width 0.25) (layer "F.Cu") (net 49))
 (segment (start 78.232 74.676) (end 74.580511 71.024511) (width 0.25) (layer "F.Cu") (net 50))
 (segment (start 74.580511 71.024511) (end 62.134511 71.024511) (width 0.25) (layer "F.Cu") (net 50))
 (segment (start 86.657 85.301) (end 86.614 85.344) (width 0.25) (layer "F.Cu") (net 50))
 (segment (start 88.764 85.301) (end 86.657 85.301) (width 0.25) (layer "F.Cu") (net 50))
 (segment (start 62.134511 71.024511) (end 60.96 69.85) (width 0.25) (layer "F.Cu") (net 50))
 (via (at 86.614 85.344) (size 0.8) (drill 0.4) (layers "F.Cu" "B.Cu") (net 50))
 (via (at 78.232 74.676) (size 0.8) (drill 0.4) (layers "F.Cu" "B.Cu") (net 50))
 (segment (start 86.614 85.344) (end 78.994 85.344) (width 0.25) (layer "B.Cu") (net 50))
 (segment (start 78.994 85.344) (end 78.232 84.582) (width 0.25) (layer "B.Cu") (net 50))
 (segment (start 78.232 84.582) (end 78.232 74.676) (width 0.25) (layer "B.Cu") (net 50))
 (segment (start 93.202 94.1925) (end 94.996 95.9865) (width 0.25) (layer "F.Cu") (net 20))
 (segment (start 93.202 94.168) (end 93.202 94.1925) (width 0.25) (layer "F.Cu") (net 20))
 (segment (start 93.538 92.268) (end 94.742 93.472) (width 0.25) (layer "F.Cu") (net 14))
 (segment (start 94.996 90.474) (end 93.202 92.268) (width 0.25) (layer "F.Cu") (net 14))
 (segment (start 94.996 89.9415) (end 94.996 90.474) (width 0.25) (layer "F.Cu") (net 14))
 (segment (start 93.202 92.268) (end 93.538 92.268) (width 0.25) (layer "F.Cu") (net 14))
 (via (at 94.742 93.472) (size 0.8) (drill 0.4) (layers "F.Cu" "B.Cu") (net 14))
 (via (at 101.76 103.251) (size 0.8) (drill 0.4) (layers "F.Cu" "B.Cu") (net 14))
 (segment (start 94.742 93.472) (end 101.76 100.49) (width 0.25) (layer "B.Cu") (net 14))
 (segment (start 101.76 100.49) (end 101.76 103.251) (width 0.25) (layer "B.Cu") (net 14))
 (segment (start 89.593022 95.461) (end 88.764 95.461) (width 0.25) (layer "F.Cu") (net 51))
 (segment (start 91.202 93.218) (end 91.202 93.852022) (width 0.25) (layer "F.Cu") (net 51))
 (segment (start 91.202 93.852022) (end 89.593022 95.461) (width 0.25) (layer "F.Cu") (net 51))
 (segment (start 94.9555 88.326) (end 94.996 88.3665) (width 0.25) (layer "F.Cu") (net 18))
 (segment (start 93.202 88.326) (end 94.9555 88.326) (width 0.25) (layer "F.Cu") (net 18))
 (segment (start 94.298799 86.426) (end 95.79552 87.922721) (width 0.25) (layer "F.Cu") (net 13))
 (segment (start 95.79552 96.76198) (end 94.996 97.5615) (width 0.25) (layer "F.Cu") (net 13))
 (segment (start 95.79552 87.922721) (end 95.79552 96.76198) (width 0.25) (layer "F.Cu") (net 13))
 (segment (start 93.202 86.426) (end 94.298799 86.426) (width 0.25) (layer "F.Cu") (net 13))
 (segment (start 95.0215 97.5615) (end 96.266 98.806) (width 0.25) (layer "F.Cu") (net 13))
 (segment (start 94.996 97.5615) (end 95.0215 97.5615) (width 0.25) (layer "F.Cu") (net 13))
 (via (at 96.266 98.806) (size 0.8) (drill 0.4) (layers "F.Cu" "B.Cu") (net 13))
 (via (at 101.76 104.521) (size 0.8) (drill 0.4) (layers "F.Cu" "B.Cu") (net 13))
 (segment (start 96.266 99.027) (end 101.76 104.521) (width 0.25) (layer "B.Cu") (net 13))
 (segment (start 96.266 98.806) (end 96.266 99.027) (width 0.25) (layer "B.Cu") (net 13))
 (segment (start 78.767511 81.815511) (end 80.264 83.312) (width 0.25) (layer "F.Cu") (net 19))
 (segment (start 71.764 81.491) (end 72.088511 81.815511) (width 0.25) (layer "F.Cu") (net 19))
 (segment (start 72.088511 81.815511) (end 78.767511 81.815511) (width 0.25) (layer "F.Cu") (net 19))
 (segment (start 91.186 85.344) (end 91.186 87.36) (width 0.25) (layer "F.Cu") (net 19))
 (segment (start 91.186 87.36) (end 91.202 87.376) (width 0.25) (layer "F.Cu") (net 19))
 (via (at 91.186 85.344) (size 0.8) (drill 0.4) (layers "F.Cu" "B.Cu") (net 19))
 (via (at 80.264 83.312) (size 0.8) (drill 0.4) (layers "F.Cu" "B.Cu") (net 19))
 (segment (start 80.264 83.312) (end 89.154 83.312) (width 0.25) (layer "B.Cu") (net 19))
 (segment (start 89.154 83.312) (end 91.186 85.344) (width 0.25) (layer "B.Cu") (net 19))
 (segment (start 81.989489 93.325511) (end 90.644978 101.981) (width 0.25) (layer "F.Cu") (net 2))
 (segment (start 72.168511 93.325511) (end 81.989489 93.325511) (width 0.25) (layer "F.Cu") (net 2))
 (segment (start 90.644978 101.981) (end 96.36 101.981) (width 0.25) (layer "F.Cu") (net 2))
 (segment (start 71.764 92.921) (end 72.168511 93.325511) (width 0.25) (layer "F.Cu") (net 2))
 (segment (start 81.653022 103.251) (end 72.593022 94.191) (width 0.25) (layer "F.Cu") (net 3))
 (segment (start 72.593022 94.191) (end 71.764 94.191) (width 0.25) (layer "F.Cu") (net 3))
 (segment (start 96.36 103.251) (end 81.653022 103.251) (width 0.25) (layer "F.Cu") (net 3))
 (segment (start 62.325489 96.615489) (end 60.96 95.25) (width 0.25) (layer "F.Cu") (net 34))
 (segment (start 71.648489 96.615489) (end 62.325489 96.615489) (width 0.25) (layer "F.Cu") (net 34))
 (segment (start 71.764 96.731) (end 71.648489 96.615489) (width 0.25) (layer "F.Cu") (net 34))
 (segment (start 71.764 95.461) (end 66.251 95.461) (width 0.25) (layer "F.Cu") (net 35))
 (segment (start 66.251 95.461) (end 63.5 92.71) (width 0.25) (layer "F.Cu") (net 35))
 (segment (start 71.764 91.651) (end 71.648489 91.535489) (width 0.25) (layer "F.Cu") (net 36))
 (segment (start 62.134511 91.535489) (end 60.96 92.71) (width 0.25) (layer "F.Cu") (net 36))
 (segment (start 71.648489 91.535489) (end 62.134511 91.535489) (width 0.25) (layer "F.Cu") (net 36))
 (segment (start 71.764 89.111) (end 64.559 89.111) (width 0.25) (layer "F.Cu") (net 37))
 (segment (start 64.559 89.111) (end 63.5 90.17) (width 0.25) (layer "F.Cu") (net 37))
 (segment (start 64.95001 87.841) (end 63.986499 88.804511) (width 0.25) (layer "F.Cu") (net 38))
 (segment (start 71.764 87.841) (end 64.95001 87.841) (width 0.25) (layer "F.Cu") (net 38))
 (segment (start 62.325489 88.804511) (end 60.96 90.17) (width 0.25) (layer "F.Cu") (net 38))
 (segment (start 63.986499 88.804511) (end 62.325489 88.804511) (width 0.25) (layer "F.Cu") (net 38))
 (segment (start 71.764 86.571) (end 64.559 86.571) (width 0.25) (layer "F.Cu") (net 39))
 (segment (start 64.559 86.571) (end 63.5 87.63) (width 0.25) (layer "F.Cu") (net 39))
 (segment (start 63.986499 86.264511) (end 62.325489 86.264511) (width 0.25) (layer "F.Cu") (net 40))
 (segment (start 64.95001 85.301) (end 63.986499 86.264511) (width 0.25) (layer "F.Cu") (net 40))
 (segment (start 71.764 85.301) (end 64.95001 85.301) (width 0.25) (layer "F.Cu") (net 40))
 (segment (start 62.325489 86.264511) (end 60.96 87.63) (width 0.25) (layer "F.Cu") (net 40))
 (segment (start 71.764 84.031) (end 64.559 84.031) (width 0.25) (layer "F.Cu") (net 41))
 (segment (start 64.559 84.031) (end 63.5 85.09) (width 0.25) (layer "F.Cu") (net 41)))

